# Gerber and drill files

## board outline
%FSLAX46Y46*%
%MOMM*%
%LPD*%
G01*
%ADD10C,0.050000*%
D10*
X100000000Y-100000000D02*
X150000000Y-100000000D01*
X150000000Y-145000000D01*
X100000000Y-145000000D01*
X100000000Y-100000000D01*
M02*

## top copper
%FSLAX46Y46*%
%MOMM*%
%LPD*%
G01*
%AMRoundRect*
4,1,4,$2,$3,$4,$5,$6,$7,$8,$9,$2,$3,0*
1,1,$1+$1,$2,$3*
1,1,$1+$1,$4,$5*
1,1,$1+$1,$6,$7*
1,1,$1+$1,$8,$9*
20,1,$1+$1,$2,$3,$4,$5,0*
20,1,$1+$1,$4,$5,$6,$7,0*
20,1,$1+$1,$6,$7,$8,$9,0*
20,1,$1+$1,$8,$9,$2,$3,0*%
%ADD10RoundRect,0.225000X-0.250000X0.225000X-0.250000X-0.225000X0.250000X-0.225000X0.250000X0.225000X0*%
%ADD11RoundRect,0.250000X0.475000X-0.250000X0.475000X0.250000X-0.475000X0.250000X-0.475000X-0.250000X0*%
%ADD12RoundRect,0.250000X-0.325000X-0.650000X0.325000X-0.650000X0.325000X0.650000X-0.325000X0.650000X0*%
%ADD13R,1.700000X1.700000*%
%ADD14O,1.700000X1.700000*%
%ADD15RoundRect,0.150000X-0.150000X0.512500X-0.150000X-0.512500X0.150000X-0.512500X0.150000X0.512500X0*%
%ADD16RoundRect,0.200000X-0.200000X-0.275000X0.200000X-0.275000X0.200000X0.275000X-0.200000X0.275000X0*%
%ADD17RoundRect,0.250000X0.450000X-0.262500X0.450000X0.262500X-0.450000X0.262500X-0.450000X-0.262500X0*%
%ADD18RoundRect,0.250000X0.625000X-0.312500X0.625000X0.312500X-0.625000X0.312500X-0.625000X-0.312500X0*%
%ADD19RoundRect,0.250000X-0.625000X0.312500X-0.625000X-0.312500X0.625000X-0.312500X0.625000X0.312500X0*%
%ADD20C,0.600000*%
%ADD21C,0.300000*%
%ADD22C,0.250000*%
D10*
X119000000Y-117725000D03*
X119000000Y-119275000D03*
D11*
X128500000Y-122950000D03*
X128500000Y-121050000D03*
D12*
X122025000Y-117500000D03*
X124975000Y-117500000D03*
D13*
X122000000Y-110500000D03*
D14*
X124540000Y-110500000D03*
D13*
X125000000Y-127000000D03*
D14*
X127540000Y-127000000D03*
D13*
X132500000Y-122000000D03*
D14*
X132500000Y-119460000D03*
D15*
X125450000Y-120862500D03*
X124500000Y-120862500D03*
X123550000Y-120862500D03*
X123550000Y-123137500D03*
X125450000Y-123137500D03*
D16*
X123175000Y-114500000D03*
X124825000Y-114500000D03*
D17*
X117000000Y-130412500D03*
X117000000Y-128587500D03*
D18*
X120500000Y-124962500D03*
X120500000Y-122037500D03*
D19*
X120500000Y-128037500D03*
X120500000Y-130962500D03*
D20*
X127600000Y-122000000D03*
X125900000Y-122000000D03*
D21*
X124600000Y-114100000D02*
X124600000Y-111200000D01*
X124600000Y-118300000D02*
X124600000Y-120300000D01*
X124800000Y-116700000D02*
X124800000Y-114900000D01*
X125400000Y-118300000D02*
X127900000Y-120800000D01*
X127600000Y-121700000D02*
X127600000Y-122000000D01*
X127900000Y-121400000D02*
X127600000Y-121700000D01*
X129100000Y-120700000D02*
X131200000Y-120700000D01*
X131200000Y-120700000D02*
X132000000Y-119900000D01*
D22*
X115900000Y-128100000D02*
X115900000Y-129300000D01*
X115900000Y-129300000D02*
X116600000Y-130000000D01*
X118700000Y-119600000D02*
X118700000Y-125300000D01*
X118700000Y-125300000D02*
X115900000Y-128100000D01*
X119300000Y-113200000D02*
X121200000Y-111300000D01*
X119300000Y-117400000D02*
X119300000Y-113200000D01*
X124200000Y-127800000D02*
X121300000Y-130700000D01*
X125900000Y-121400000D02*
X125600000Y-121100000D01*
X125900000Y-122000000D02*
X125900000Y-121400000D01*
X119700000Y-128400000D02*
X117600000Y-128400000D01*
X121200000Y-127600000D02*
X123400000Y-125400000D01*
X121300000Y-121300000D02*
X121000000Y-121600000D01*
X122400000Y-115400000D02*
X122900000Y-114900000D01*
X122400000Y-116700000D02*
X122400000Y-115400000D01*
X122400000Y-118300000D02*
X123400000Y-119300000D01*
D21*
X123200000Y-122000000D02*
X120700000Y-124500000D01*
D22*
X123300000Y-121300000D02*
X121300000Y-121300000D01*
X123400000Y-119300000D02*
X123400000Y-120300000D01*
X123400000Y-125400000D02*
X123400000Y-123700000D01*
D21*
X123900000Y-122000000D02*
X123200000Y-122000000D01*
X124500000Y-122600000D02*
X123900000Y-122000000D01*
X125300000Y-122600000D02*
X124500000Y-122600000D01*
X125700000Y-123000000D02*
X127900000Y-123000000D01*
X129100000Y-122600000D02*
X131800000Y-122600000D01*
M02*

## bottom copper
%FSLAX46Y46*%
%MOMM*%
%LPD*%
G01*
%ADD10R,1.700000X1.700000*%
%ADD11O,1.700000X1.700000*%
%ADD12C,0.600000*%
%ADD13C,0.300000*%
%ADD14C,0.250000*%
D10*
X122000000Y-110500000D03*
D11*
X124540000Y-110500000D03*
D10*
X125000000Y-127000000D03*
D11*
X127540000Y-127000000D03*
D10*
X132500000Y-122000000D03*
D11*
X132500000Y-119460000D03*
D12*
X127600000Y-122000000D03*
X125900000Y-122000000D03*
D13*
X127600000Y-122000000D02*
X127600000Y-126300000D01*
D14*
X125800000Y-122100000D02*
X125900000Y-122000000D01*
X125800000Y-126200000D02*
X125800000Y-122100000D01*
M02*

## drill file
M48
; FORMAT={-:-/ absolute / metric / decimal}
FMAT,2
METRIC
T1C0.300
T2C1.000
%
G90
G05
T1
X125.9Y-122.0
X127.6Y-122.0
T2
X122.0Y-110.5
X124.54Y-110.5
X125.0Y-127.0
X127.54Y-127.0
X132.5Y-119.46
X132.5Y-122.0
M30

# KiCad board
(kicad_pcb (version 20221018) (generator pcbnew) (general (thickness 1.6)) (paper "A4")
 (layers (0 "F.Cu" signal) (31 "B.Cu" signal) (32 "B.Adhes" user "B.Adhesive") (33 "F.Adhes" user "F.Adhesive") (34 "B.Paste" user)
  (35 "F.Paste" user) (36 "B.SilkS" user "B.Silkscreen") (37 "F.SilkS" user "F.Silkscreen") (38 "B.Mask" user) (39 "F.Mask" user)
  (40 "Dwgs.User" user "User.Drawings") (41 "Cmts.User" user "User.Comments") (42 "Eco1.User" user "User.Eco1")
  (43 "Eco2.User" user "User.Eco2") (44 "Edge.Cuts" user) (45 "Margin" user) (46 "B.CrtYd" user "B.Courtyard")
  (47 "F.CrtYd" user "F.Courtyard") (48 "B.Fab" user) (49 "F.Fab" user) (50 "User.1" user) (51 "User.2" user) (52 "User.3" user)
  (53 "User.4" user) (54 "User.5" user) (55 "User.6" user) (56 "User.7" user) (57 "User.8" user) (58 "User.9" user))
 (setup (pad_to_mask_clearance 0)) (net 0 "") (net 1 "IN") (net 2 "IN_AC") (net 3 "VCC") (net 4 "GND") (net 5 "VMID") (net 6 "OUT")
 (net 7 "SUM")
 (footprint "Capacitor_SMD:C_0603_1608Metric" (layer "F.Cu") (at 119 118.5 -90)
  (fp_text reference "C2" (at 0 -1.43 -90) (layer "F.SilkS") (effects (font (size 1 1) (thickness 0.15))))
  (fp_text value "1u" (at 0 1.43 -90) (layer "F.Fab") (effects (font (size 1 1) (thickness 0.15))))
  (pad "1" smd roundrect (at -0.775 0 270) (size 0.9 0.95) (layers "F.Cu" "F.Paste" "F.Mask") (roundrect_rratio 0.25) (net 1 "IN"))
  (pad "2" smd roundrect (at 0.775 0 270) (size 0.9 0.95) (layers "F.Cu" "F.Paste" "F.Mask") (roundrect_rratio 0.25) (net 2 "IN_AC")))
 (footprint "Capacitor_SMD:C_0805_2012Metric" (layer "F.Cu") (at 128.5 122 90)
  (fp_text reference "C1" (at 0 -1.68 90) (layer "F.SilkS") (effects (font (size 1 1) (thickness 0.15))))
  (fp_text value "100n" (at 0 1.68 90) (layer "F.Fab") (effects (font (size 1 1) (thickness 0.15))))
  (pad "1" smd roundrect (at -0.95 0 90) (size 1 1.45) (layers "F.Cu" "F.Paste" "F.Mask") (roundrect_rratio 0.25) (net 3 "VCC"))
  (pad "2" smd roundrect (at 0.95 0 90) (size 1 1.45) (layers "F.Cu" "F.Paste" "F.Mask") (roundrect_rratio 0.25) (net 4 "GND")))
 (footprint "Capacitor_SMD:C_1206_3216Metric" (layer "F.Cu") (at 123.5 117.5)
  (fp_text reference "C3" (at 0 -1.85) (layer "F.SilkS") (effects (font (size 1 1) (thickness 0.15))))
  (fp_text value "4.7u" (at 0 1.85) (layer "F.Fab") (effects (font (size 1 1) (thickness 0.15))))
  (pad "1" smd roundrect (at -1.475 0) (size 1.15 1.8) (layers "F.Cu" "F.Paste" "F.Mask") (roundrect_rratio 0.217391) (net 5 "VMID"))
  (pad "2" smd roundrect (at 1.475 0) (size 1.15 1.8) (layers "F.Cu" "F.Paste" "F.Mask") (roundrect_rratio 0.217391) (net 4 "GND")))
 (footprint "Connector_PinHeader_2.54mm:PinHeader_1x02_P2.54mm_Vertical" (layer "F.Cu") (at 122 110.5 90)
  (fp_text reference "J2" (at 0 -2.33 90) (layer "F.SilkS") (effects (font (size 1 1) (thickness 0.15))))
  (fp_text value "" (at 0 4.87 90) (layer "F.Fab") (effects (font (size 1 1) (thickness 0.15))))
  (pad "1" thru_hole rect (at 0 0 90) (size 1.7 1.7) (drill 1) (layers "*.Cu" "*.Mask") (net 1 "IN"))
  (pad "2" thru_hole oval (at 0 2.54 90) (size 1.7 1.7) (drill 1) (layers "*.Cu" "*.Mask") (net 4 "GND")))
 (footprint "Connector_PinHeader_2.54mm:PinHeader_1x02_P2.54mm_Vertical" (layer "F.Cu") (at 125 127 90)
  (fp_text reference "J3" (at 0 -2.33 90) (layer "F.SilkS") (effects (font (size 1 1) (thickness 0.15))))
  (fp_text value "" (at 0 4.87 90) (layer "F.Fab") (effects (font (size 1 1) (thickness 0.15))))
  (pad "1" thru_hole rect (at 0 0 90) (size 1.7 1.7) (drill 1) (layers "*.Cu" "*.Mask") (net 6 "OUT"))
  (pad "2" thru_hole oval (at 0 2.54 90) (size 1.7 1.7) (drill 1) (layers "*.Cu" "*.Mask") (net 4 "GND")))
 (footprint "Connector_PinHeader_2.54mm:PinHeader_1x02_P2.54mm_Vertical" (layer "F.Cu") (at 132.5 122 180)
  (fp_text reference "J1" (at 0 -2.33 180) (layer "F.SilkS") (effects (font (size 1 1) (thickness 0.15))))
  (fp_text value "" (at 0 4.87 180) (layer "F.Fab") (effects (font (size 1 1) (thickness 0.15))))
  (pad "1" thru_hole rect (at 0 0 180) (size 1.7 1.7) (drill 1) (layers "*.Cu" "*.Mask") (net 3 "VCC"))
  (pad "2" thru_hole oval (at 0 2.54 180) (size 1.7 1.7) (drill 1) (layers "*.Cu" "*.Mask") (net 4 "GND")))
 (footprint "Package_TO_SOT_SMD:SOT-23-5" (layer "F.Cu") (at 124.5 122 -90)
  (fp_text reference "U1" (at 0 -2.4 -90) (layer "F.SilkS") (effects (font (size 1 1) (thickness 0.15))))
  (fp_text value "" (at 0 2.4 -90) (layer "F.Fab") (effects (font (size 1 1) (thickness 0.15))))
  (pad "1" smd roundrect (at -1.1375 -0.95 270) (size 1.325 0.6) (layers "F.Cu" "F.Paste" "F.Mask") (roundrect_rratio 0.25) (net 6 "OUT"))
  (pad "2" smd roundrect (at -1.1375 0 270) (size 1.325 0.6) (layers "F.Cu" "F.Paste" "F.Mask") (roundrect_rratio 0.25) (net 4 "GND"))
  (pad "3" smd roundrect (at -1.1375 0.95 270) (size 1.325 0.6) (layers "F.Cu" "F.Paste" "F.Mask") (roundrect_rratio 0.25) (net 5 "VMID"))
  (pad "4" smd roundrect (at 1.1375 0.95 270) (size 1.325 0.6) (layers "F.Cu" "F.Paste" "F.Mask") (roundrect_rratio 0.25) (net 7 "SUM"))
  (pad "5" smd roundrect (at 1.1375 -0.95 270) (size 1.325 0.6) (layers "F.Cu" "F.Paste" "F.Mask") (roundrect_rratio 0.25) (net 3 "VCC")))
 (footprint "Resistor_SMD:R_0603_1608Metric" (layer "F.Cu") (at 124 114.5)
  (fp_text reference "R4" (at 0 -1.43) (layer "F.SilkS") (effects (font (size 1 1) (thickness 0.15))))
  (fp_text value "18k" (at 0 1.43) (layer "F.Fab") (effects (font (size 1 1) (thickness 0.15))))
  (pad "1" smd roundrect (at -0.825 0) (size 0.8 0.95) (layers "F.Cu" "F.Paste" "F.Mask") (roundrect_rratio 0.25) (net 5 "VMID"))
  (pad "2" smd roundrect (at 0.825 0) (size 0.8 0.95) (layers "F.Cu" "F.Paste" "F.Mask") (roundrect_rratio 0.25) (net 4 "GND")))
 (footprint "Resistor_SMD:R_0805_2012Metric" (layer "F.Cu") (at 117 129.5 90)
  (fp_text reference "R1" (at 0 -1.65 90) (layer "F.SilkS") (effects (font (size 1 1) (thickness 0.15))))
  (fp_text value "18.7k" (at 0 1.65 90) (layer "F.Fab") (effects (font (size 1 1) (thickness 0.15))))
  (pad "1" smd roundrect (at -0.9125 0 90) (size 1.025 1.4) (layers "F.Cu" "F.Paste" "F.Mask") (roundrect_rratio 0.243902) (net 2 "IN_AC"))
  (pad "2" smd roundrect (at 0.9125 0 90) (size 1.025 1.4) (layers "F.Cu" "F.Paste" "F.Mask") (roundrect_rratio 0.243902) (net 7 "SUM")))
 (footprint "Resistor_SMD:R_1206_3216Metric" (layer "F.Cu") (at 120.5 123.5 90)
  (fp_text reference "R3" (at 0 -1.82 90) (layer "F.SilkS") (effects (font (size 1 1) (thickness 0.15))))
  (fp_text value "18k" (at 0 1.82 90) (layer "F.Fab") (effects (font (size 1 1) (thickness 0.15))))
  (pad "1" smd roundrect (at -1.4625 0 90) (size 1.125 1.75) (layers "F.Cu" "F.Paste" "F.Mask") (roundrect_rratio 0.222222) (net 3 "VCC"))
  (pad "2" smd roundrect (at 1.4625 0 90) (size 1.125 1.75) (layers "F.Cu" "F.Paste" "F.Mask") (roundrect_rratio 0.222222) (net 5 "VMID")))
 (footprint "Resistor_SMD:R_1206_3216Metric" (layer "F.Cu") (at 120.5 129.5 -90)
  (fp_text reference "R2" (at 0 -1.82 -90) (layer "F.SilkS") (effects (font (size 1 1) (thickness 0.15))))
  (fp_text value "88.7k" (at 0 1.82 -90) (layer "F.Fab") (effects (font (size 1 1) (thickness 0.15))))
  (pad "1" smd roundrect (at -1.4625 0 270) (size 1.125 1.75) (layers "F.Cu" "F.Paste" "F.Mask") (roundrect_rratio 0.222222) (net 7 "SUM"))
  (pad "2" smd roundrect (at 1.4625 0 270) (size 1.125 1.75) (layers "F.Cu" "F.Paste" "F.Mask") (roundrect_rratio 0.222222) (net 6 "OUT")))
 (gr_rect (start 100 100) (end 150 145) (stroke (width 0.05) (type default)) (fill none) (layer "Edge.Cuts"))
 (segment (start 124.6 114.1) (end 124.6 111.2) (width 0.3) (layer "F.Cu") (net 4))
 (segment (start 124.6 118.3) (end 124.6 120.3) (width 0.3) (layer "F.Cu") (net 4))
 (segment (start 124.8 116.7) (end 124.8 114.9) (width 0.3) (layer "F.Cu") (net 4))
 (segment (start 125.4 118.3) (end 127.9 120.8) (width 0.3) (layer "F.Cu") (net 4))
 (segment (start 127.6 121.7) (end 127.6 122) (width 0.3) (layer "F.Cu") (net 4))
 (segment (start 127.9 121.4) (end 127.6 121.7) (width 0.3) (layer "F.Cu") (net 4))
 (segment (start 129.1 120.7) (end 131.2 120.7) (width 0.3) (layer "F.Cu") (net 4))
 (segment (start 131.2 120.7) (end 132 119.9) (width 0.3) (layer "F.Cu") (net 4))
 (via (at 127.6 122) (size 0.6) (drill 0.3) (layers "F.Cu" "B.Cu") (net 4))
 (segment (start 115.9 128.1) (end 115.9 129.3) (width 0.25) (layer "F.Cu") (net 2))
 (segment (start 115.9 129.3) (end 116.6 130) (width 0.25) (layer "F.Cu") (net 2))
 (segment (start 118.7 119.6) (end 118.7 125.3) (width 0.25) (layer "F.Cu") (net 2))
 (segment (start 118.7 125.3) (end 115.9 128.1) (width 0.25) (layer "F.Cu") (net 2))
 (segment (start 119.3 113.2) (end 121.2 111.3) (width 0.25) (layer "F.Cu") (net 1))
 (segment (start 119.3 117.4) (end 119.3 113.2) (width 0.25) (layer "F.Cu") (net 1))
 (segment (start 124.2 127.8) (end 121.3 130.7) (width 0.25) (layer "F.Cu") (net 6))
 (segment (start 125.9 121.4) (end 125.6 121.1) (width 0.25) (layer "F.Cu") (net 6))
 (segment (start 125.9 122) (end 125.9 121.4) (width 0.25) (layer "F.Cu") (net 6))
 (segment (start 127.6 122) (end 127.6 126.3) (width 0.3) (layer "B.Cu") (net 4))
 (via (at 125.9 122) (size 0.6) (drill 0.3) (layers "F.Cu" "B.Cu") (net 6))
 (segment (start 119.7 128.4) (end 117.6 128.4) (width 0.25) (layer "F.Cu") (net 7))
 (segment (start 121.2 127.6) (end 123.4 125.4) (width 0.25) (layer "F.Cu") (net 7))
 (segment (start 121.3 121.3) (end 121 121.6) (width 0.25) (layer "F.Cu") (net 5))
 (segment (start 122.4 115.4) (end 122.9 114.9) (width 0.25) (layer "F.Cu") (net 5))
 (segment (start 122.4 116.7) (end 122.4 115.4) (width 0.25) (layer "F.Cu") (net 5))
 (segment (start 122.4 118.3) (end 123.4 119.3) (width 0.25) (layer "F.Cu") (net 5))
 (segment (start 123.2 122) (end 120.7 124.5) (width 0.3) (layer "F.Cu") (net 3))
 (segment (start 123.3 121.3) (end 121.3 121.3) (width 0.25) (layer "F.Cu") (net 5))
 (segment (start 123.4 119.3) (end 123.4 120.3) (width 0.25) (layer "F.Cu") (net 5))
 (segment (start 123.4 125.4) (end 123.4 123.7) (width 0.25) (layer "F.Cu") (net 7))
 (segment (start 123.9 122) (end 123.2 122) (width 0.3) (layer "F.Cu") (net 3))
 (segment (start 124.5 122.6) (end 123.9 122) (width 0.3) (layer "F.Cu") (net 3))
 (segment (start 125.3 122.6) (end 124.5 122.6) (width 0.3) (layer "F.Cu") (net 3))
 (segment (start 125.7 123) (end 127.9 123) (width 0.3) (layer "F.Cu") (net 3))
 (segment (start 125.8 122.1) (end 125.9 122) (width 0.25) (layer "B.Cu") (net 6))
 (segment (start 125.8 126.2) (end 125.8 122.1) (width 0.25) (layer "B.Cu") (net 6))
 (segment (start 129.1 122.6) (end 131.8 122.6) (width 0.3) (layer "F.Cu") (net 3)))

